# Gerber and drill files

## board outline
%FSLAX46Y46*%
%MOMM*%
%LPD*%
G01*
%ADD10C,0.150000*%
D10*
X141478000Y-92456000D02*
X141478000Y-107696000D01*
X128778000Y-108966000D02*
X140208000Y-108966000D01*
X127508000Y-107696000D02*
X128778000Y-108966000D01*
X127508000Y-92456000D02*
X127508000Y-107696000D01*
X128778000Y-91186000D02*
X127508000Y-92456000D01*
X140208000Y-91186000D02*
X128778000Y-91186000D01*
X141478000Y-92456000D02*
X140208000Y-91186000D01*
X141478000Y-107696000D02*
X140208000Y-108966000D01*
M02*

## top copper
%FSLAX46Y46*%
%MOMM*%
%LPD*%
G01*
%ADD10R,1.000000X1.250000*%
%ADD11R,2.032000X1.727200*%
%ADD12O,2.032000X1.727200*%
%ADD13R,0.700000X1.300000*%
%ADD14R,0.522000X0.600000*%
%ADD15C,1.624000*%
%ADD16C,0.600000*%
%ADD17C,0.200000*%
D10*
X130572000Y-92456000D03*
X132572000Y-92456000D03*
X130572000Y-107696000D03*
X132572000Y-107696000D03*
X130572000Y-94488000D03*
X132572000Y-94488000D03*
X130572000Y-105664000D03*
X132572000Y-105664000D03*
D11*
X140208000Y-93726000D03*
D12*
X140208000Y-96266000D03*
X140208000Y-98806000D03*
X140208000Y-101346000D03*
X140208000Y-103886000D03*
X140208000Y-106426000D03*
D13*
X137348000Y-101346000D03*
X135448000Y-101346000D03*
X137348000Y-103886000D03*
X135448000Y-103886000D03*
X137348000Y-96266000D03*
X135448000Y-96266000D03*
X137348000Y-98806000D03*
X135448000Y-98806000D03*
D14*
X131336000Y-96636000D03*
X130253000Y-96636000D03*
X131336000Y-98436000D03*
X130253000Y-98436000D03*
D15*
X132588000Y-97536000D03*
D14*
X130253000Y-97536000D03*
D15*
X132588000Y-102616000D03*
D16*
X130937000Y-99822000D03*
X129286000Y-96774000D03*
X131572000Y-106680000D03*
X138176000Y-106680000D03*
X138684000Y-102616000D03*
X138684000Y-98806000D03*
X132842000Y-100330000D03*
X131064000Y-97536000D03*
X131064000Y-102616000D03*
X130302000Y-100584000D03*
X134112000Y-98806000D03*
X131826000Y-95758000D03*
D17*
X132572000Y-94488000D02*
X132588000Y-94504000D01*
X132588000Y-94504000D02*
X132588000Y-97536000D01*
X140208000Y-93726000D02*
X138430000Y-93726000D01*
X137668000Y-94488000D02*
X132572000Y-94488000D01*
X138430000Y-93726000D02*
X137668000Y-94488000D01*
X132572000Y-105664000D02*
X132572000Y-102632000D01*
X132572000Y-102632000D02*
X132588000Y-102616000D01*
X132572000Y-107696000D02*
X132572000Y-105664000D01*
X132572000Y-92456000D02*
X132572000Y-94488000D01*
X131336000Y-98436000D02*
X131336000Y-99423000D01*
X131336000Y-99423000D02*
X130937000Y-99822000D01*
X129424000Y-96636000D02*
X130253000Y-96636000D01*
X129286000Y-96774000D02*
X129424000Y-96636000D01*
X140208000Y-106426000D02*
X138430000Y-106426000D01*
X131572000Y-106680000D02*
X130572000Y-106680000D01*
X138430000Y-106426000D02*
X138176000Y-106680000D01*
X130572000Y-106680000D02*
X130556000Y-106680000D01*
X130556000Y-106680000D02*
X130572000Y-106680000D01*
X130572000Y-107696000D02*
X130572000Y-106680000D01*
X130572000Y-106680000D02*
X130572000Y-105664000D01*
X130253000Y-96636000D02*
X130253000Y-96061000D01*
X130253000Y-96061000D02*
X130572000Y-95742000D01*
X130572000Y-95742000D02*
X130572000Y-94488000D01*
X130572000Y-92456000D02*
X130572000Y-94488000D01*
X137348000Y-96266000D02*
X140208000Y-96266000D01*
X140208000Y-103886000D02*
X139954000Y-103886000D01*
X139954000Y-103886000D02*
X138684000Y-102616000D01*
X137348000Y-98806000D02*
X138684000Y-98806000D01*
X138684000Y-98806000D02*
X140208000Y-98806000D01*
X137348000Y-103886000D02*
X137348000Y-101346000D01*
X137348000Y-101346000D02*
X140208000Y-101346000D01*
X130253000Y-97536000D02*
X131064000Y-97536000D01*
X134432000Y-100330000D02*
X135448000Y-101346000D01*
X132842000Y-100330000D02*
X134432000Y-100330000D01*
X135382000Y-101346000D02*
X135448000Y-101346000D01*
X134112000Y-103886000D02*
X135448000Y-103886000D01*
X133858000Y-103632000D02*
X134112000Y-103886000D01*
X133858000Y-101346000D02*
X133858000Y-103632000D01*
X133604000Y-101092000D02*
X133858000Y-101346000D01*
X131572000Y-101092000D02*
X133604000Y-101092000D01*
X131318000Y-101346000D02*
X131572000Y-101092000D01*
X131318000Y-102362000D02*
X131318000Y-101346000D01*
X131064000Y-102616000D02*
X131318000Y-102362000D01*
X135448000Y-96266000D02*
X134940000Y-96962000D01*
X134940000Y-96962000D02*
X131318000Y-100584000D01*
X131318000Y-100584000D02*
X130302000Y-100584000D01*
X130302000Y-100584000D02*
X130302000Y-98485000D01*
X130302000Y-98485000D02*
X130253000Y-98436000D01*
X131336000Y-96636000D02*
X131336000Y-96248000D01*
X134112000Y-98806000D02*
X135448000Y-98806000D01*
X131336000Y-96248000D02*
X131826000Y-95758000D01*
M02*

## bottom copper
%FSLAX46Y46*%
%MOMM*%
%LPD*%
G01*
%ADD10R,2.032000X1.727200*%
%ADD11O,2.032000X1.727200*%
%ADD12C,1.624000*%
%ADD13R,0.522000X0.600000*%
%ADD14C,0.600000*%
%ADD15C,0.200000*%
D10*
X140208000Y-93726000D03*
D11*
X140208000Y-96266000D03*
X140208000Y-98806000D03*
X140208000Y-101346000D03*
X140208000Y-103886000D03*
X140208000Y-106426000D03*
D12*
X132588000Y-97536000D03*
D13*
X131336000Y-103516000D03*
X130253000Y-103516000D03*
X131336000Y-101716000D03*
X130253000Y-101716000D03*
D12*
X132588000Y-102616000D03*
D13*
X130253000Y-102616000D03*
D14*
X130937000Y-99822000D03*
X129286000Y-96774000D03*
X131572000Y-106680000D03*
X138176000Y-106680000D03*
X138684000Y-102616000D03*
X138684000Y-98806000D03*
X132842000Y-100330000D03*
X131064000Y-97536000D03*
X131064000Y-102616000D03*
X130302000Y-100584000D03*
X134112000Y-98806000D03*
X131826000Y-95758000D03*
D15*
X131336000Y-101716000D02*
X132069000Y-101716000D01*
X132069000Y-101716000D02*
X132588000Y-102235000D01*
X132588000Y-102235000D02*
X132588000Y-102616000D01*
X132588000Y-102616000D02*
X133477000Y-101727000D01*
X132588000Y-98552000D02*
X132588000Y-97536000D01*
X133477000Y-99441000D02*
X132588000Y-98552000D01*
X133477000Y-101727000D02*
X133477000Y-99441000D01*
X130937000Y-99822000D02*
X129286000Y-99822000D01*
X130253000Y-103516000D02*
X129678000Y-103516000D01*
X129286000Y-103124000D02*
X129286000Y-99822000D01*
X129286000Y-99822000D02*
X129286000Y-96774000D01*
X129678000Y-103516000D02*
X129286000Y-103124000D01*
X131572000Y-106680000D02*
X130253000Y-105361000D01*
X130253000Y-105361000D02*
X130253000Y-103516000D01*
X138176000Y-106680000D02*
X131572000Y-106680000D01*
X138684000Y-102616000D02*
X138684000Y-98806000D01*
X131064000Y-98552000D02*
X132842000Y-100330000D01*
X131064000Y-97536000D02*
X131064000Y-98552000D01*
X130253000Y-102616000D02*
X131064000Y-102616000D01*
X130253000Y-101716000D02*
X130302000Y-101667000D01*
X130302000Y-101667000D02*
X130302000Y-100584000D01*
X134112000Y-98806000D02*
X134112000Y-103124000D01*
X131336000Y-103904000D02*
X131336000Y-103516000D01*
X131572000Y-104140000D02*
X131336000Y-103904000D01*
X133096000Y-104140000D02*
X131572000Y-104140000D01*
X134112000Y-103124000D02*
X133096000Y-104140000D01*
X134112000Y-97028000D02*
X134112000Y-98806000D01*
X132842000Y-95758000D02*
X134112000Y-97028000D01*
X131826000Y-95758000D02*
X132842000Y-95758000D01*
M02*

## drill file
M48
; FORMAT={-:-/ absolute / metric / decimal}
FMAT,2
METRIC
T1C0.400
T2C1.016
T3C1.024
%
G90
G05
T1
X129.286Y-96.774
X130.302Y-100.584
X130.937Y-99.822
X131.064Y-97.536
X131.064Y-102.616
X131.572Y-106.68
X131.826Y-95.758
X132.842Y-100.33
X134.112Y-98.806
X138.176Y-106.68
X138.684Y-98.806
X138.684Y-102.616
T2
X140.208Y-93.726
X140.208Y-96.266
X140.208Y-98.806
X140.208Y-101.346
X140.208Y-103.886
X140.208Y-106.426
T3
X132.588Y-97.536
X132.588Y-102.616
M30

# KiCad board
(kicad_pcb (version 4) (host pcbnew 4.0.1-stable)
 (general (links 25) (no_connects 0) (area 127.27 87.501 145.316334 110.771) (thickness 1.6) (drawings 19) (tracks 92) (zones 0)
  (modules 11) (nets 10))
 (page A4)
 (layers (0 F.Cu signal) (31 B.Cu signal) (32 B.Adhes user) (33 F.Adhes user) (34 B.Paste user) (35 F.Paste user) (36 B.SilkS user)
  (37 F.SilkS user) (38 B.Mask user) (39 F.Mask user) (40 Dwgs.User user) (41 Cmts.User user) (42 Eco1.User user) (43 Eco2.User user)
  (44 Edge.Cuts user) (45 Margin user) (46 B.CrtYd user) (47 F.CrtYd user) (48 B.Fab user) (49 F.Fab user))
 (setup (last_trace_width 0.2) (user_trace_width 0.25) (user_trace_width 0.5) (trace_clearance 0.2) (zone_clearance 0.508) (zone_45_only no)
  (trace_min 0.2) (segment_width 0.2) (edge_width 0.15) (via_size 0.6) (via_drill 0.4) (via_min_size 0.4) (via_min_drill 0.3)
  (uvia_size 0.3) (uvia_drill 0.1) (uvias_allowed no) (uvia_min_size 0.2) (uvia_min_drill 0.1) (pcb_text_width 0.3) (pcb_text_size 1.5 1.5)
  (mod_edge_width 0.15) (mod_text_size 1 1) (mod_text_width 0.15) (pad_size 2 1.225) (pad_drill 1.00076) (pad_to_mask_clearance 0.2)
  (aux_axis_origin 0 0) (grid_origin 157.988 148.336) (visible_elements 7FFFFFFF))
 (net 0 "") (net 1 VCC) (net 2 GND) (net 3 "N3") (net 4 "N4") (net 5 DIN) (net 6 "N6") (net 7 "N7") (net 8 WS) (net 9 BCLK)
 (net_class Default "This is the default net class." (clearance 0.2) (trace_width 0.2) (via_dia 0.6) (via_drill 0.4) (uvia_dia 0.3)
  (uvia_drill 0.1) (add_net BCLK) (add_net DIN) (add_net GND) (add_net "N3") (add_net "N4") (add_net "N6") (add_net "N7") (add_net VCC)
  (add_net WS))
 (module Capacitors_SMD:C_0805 (layer F.Cu) (at 131.572 92.456)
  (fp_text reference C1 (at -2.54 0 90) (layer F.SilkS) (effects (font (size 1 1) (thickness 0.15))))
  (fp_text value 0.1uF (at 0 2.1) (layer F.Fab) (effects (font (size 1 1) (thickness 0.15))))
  (pad 1 smd rect (at -1 0) (size 1 1.25) (layers F.Cu F.Paste F.Mask) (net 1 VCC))
  (pad 2 smd rect (at 1 0) (size 1 1.25) (layers F.Cu F.Paste F.Mask) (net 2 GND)))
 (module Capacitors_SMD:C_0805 (layer F.Cu) (at 131.572 107.696)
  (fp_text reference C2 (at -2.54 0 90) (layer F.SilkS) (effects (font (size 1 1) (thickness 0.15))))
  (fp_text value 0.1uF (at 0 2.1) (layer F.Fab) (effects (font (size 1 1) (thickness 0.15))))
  (pad 1 smd rect (at -1 0) (size 1 1.25) (layers F.Cu F.Paste F.Mask) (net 1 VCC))
  (pad 2 smd rect (at 1 0) (size 1 1.25) (layers F.Cu F.Paste F.Mask) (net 2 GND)))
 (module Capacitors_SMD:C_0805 (layer F.Cu) (at 131.572 94.488)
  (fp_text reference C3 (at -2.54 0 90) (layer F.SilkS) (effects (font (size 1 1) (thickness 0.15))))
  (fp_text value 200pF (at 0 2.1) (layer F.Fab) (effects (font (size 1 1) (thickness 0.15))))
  (pad 1 smd rect (at -1 0) (size 1 1.25) (layers F.Cu F.Paste F.Mask) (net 1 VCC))
  (pad 2 smd rect (at 1 0) (size 1 1.25) (layers F.Cu F.Paste F.Mask) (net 2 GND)))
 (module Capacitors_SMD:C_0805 (layer F.Cu) (at 131.572 105.664)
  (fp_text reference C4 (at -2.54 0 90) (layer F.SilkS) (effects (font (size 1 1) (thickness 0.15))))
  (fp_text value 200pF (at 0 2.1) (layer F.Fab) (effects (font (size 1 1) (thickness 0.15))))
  (pad 1 smd rect (at -1 0) (size 1 1.25) (layers F.Cu F.Paste F.Mask) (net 1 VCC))
  (pad 2 smd rect (at 1 0) (size 1 1.25) (layers F.Cu F.Paste F.Mask) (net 2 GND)))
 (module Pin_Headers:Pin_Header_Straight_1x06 (layer F.Cu) (at 140.208 93.726)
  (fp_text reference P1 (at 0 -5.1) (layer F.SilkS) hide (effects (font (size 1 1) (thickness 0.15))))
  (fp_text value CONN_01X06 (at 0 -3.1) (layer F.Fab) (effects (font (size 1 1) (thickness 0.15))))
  (pad 1 thru_hole rect (at 0 0) (size 2.032 1.7272) (drill 1.016) (layers *.Cu *.Mask F.SilkS) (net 2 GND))
  (pad 2 thru_hole oval (at 0 2.54) (size 2.032 1.7272) (drill 1.016) (layers *.Cu *.Mask F.SilkS) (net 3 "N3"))
  (pad 3 thru_hole oval (at 0 5.08) (size 2.032 1.7272) (drill 1.016) (layers *.Cu *.Mask F.SilkS) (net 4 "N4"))
  (pad 4 thru_hole oval (at 0 7.62) (size 2.032 1.7272) (drill 1.016) (layers *.Cu *.Mask F.SilkS) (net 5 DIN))
  (pad 5 thru_hole oval (at 0 10.16) (size 2.032 1.7272) (drill 1.016) (layers *.Cu *.Mask F.SilkS) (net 4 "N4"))
  (pad 6 thru_hole oval (at 0 12.7) (size 2.032 1.7272) (drill 1.016) (layers *.Cu *.Mask F.SilkS) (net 1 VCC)))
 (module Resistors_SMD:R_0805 (layer F.Cu) (at 136.398 101.346 180)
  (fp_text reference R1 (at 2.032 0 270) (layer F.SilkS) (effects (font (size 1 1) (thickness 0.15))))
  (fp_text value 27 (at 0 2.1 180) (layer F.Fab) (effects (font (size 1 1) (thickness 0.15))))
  (pad 1 smd rect (at -0.95 0 180) (size 0.7 1.3) (layers F.Cu F.Paste F.Mask) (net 5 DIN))
  (pad 2 smd rect (at 0.95 0 180) (size 0.7 1.3) (layers F.Cu F.Paste F.Mask) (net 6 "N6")))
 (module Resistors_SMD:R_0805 (layer F.Cu) (at 136.398 103.886 180)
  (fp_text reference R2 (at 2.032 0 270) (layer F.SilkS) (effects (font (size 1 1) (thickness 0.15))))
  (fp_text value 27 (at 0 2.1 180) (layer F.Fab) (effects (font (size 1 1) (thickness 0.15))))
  (pad 1 smd rect (at -0.95 0 180) (size 0.7 1.3) (layers F.Cu F.Paste F.Mask) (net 5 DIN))
  (pad 2 smd rect (at 0.95 0 180) (size 0.7 1.3) (layers F.Cu F.Paste F.Mask) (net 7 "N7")))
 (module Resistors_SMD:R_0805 (layer F.Cu) (at 136.398 96.266 180)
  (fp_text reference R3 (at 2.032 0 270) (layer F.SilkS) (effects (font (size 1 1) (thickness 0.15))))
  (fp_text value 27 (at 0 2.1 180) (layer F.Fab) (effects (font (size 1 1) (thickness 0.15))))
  (pad 1 smd rect (at -0.95 0 180) (size 0.7 1.3) (layers F.Cu F.Paste F.Mask) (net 3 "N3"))
  (pad 2 smd rect (at 0.95 0 180) (size 0.7 1.3) (layers F.Cu F.Paste F.Mask) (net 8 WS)))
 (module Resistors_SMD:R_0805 (layer F.Cu) (at 136.398 98.806 180)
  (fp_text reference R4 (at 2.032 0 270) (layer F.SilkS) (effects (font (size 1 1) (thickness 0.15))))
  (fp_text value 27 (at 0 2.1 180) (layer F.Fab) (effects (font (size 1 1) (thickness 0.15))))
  (pad 1 smd rect (at -0.95 0 180) (size 0.7 1.3) (layers F.Cu F.Paste F.Mask) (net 4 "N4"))
  (pad 2 smd rect (at 0.95 0 180) (size 0.7 1.3) (layers F.Cu F.Paste F.Mask) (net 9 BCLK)))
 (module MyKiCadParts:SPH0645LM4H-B (layer F.Cu) (at 132.588 97.536 90)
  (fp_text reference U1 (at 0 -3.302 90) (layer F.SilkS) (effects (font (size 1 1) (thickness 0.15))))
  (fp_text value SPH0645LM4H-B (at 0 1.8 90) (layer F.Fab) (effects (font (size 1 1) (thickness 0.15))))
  (pad 4 smd rect (at 0.9 -1.252 90) (size 0.6 0.522) (layers F.Cu F.Paste F.Mask) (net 9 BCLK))
  (pad 5 smd rect (at 0.9 -2.335 90) (size 0.6 0.522) (layers F.Cu F.Paste F.Mask) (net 1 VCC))
  (pad 2 smd rect (at -0.9 -1.252 90) (size 0.6 0.522) (layers F.Cu F.Paste F.Mask) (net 1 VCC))
  (pad 1 smd rect (at -0.9 -2.335 90) (size 0.6 0.522) (layers F.Cu F.Paste F.Mask) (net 8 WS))
  (pad 3 thru_hole circle (at 0 0 90) (size 1.624 1.624) (drill 1.024) (layers *.Cu *.Mask F.SilkS) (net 2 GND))
  (pad 6 smd rect (at 0 -2.335 90) (size 0.6 0.522) (layers F.Cu F.Paste F.Mask) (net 6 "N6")))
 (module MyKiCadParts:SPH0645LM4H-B (layer B.Cu) (at 132.588 102.616 270)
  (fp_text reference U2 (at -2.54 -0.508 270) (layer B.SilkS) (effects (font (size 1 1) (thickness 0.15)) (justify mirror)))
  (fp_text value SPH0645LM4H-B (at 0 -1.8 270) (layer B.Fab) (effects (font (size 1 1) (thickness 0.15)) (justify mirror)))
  (pad 4 smd rect (at 0.9 1.252 270) (size 0.6 0.522) (layers B.Cu B.Paste B.Mask) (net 9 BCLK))
  (pad 5 smd rect (at 0.9 2.335 270) (size 0.6 0.522) (layers B.Cu B.Paste B.Mask) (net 1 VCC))
  (pad 2 smd rect (at -0.9 1.252 270) (size 0.6 0.522) (layers B.Cu B.Paste B.Mask) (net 2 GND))
  (pad 1 smd rect (at -0.9 2.335 270) (size 0.6 0.522) (layers B.Cu B.Paste B.Mask) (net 8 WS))
  (pad 3 thru_hole circle (at 0 0 270) (size 1.624 1.624) (drill 1.024) (layers *.Cu *.Mask B.SilkS) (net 2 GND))
  (pad 6 smd rect (at 0 2.335 270) (size 0.6 0.522) (layers B.Cu B.Paste B.Mask) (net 7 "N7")))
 (gr_line (start 141.478 92.456) (end 141.478 107.696) (angle 90) (layer Edge.Cuts) (width 0.15))
 (gr_line (start 128.778 108.966) (end 140.208 108.966) (angle 90) (layer Edge.Cuts) (width 0.15))
 (gr_line (start 127.508 107.696) (end 128.778 108.966) (angle 90) (layer Edge.Cuts) (width 0.15))
 (gr_line (start 127.508 92.456) (end 127.508 107.696) (angle 90) (layer Edge.Cuts) (width 0.15))
 (gr_line (start 128.778 91.186) (end 127.508 92.456) (angle 90) (layer Edge.Cuts) (width 0.15))
 (gr_line (start 140.208 91.186) (end 128.778 91.186) (angle 90) (layer Edge.Cuts) (width 0.15))
 (gr_line (start 141.478 92.456) (end 140.208 91.186) (angle 90) (layer Edge.Cuts) (width 0.15))
 (gr_line (start 141.478 107.696) (end 140.208 108.966) (angle 90) (layer Edge.Cuts) (width 0.15))
 (segment (start 131.336 101.716) (end 132.069 101.716) (width 0.2) (layer B.Cu) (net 2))
 (segment (start 132.069 101.716) (end 132.588 102.235) (width 0.2) (layer B.Cu) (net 2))
 (segment (start 132.588 102.235) (end 132.588 102.616) (width 0.2) (layer B.Cu) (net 2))
 (segment (start 132.588 102.616) (end 133.477 101.727) (width 0.2) (layer B.Cu) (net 2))
 (segment (start 132.588 98.552) (end 132.588 97.536) (width 0.2) (layer B.Cu) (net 2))
 (segment (start 133.477 99.441) (end 132.588 98.552) (width 0.2) (layer B.Cu) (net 2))
 (segment (start 133.477 101.727) (end 133.477 99.441) (width 0.2) (layer B.Cu) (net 2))
 (segment (start 132.572 94.488) (end 132.588 94.504) (width 0.2) (layer F.Cu) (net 2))
 (segment (start 132.588 94.504) (end 132.588 97.536) (width 0.2) (layer F.Cu) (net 2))
 (segment (start 140.208 93.726) (end 138.43 93.726) (width 0.2) (layer F.Cu) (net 2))
 (segment (start 137.668 94.488) (end 132.572 94.488) (width 0.2) (layer F.Cu) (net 2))
 (segment (start 138.43 93.726) (end 137.668 94.488) (width 0.2) (layer F.Cu) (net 2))
 (segment (start 132.572 105.664) (end 132.572 102.632) (width 0.2) (layer F.Cu) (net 2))
 (segment (start 132.572 102.632) (end 132.588 102.616) (width 0.2) (layer F.Cu) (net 2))
 (segment (start 132.572 107.696) (end 132.572 105.664) (width 0.2) (layer F.Cu) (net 2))
 (segment (start 132.572 92.456) (end 132.572 94.488) (width 0.2) (layer F.Cu) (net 2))
 (segment (start 131.336 98.436) (end 131.336 99.423) (width 0.2) (layer F.Cu) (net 1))
 (segment (start 130.937 99.822) (end 129.286 99.822) (width 0.2) (layer B.Cu) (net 1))
 (via (at 130.937 99.822) (size 0.6) (drill 0.4) (layers F.Cu B.Cu) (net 1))
 (segment (start 131.336 99.423) (end 130.937 99.822) (width 0.2) (layer F.Cu) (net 1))
 (segment (start 130.253 103.516) (end 129.678 103.516) (width 0.2) (layer B.Cu) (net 1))
 (segment (start 129.424 96.636) (end 130.253 96.636) (width 0.2) (layer F.Cu) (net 1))
 (segment (start 129.286 96.774) (end 129.424 96.636) (width 0.2) (layer F.Cu) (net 1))
 (via (at 129.286 96.774) (size 0.6) (drill 0.4) (layers F.Cu B.Cu) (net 1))
 (segment (start 129.286 103.124) (end 129.286 99.822) (width 0.2) (layer B.Cu) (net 1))
 (segment (start 129.286 99.822) (end 129.286 96.774) (width 0.2) (layer B.Cu) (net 1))
 (segment (start 129.678 103.516) (end 129.286 103.124) (width 0.2) (layer B.Cu) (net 1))
 (segment (start 131.572 106.68) (end 130.253 105.361) (width 0.2) (layer B.Cu) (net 1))
 (segment (start 130.253 105.361) (end 130.253 103.516) (width 0.2) (layer B.Cu) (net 1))
 (segment (start 140.208 106.426) (end 138.43 106.426) (width 0.2) (layer F.Cu) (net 1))
 (segment (start 131.572 106.68) (end 130.572 106.68) (width 0.2) (layer F.Cu) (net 1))
 (via (at 131.572 106.68) (size 0.6) (drill 0.4) (layers F.Cu B.Cu) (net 1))
 (segment (start 138.176 106.68) (end 131.572 106.68) (width 0.2) (layer B.Cu) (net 1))
 (via (at 138.176 106.68) (size 0.6) (drill 0.4) (layers F.Cu B.Cu) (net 1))
 (segment (start 138.43 106.426) (end 138.176 106.68) (width 0.2) (layer F.Cu) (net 1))
 (segment (start 130.572 106.68) (end 130.556 106.68) (width 0.2) (layer F.Cu) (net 1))
 (segment (start 130.556 106.68) (end 130.572 106.68) (width 0.2) (layer F.Cu) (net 1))
 (segment (start 130.572 107.696) (end 130.572 106.68) (width 0.2) (layer F.Cu) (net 1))
 (segment (start 130.572 106.68) (end 130.572 105.664) (width 0.2) (layer F.Cu) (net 1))
 (segment (start 130.253 96.636) (end 130.253 96.061) (width 0.2) (layer F.Cu) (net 1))
 (segment (start 130.253 96.061) (end 130.572 95.742) (width 0.2) (layer F.Cu) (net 1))
 (segment (start 130.572 95.742) (end 130.572 94.488) (width 0.2) (layer F.Cu) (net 1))
 (segment (start 130.572 92.456) (end 130.572 94.488) (width 0.2) (layer F.Cu) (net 1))
 (segment (start 137.348 96.266) (end 140.208 96.266) (width 0.2) (layer F.Cu) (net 3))
 (segment (start 140.208 103.886) (end 139.954 103.886) (width 0.2) (layer F.Cu) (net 4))
 (segment (start 139.954 103.886) (end 138.684 102.616) (width 0.2) (layer F.Cu) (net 4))
 (via (at 138.684 102.616) (size 0.6) (drill 0.4) (layers F.Cu B.Cu) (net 4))
 (segment (start 138.684 102.616) (end 138.684 98.806) (width 0.2) (layer B.Cu) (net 4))
 (via (at 138.684 98.806) (size 0.6) (drill 0.4) (layers F.Cu B.Cu) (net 4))
 (segment (start 137.348 98.806) (end 138.684 98.806) (width 0.2) (layer F.Cu) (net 4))
 (segment (start 138.684 98.806) (end 140.208 98.806) (width 0.2) (layer F.Cu) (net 4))
 (segment (start 137.348 103.886) (end 137.348 101.346) (width 0.2) (layer F.Cu) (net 5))
 (segment (start 137.348 101.346) (end 140.208 101.346) (width 0.2) (layer F.Cu) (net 5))
 (segment (start 130.253 97.536) (end 131.064 97.536) (width 0.2) (layer F.Cu) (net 6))
 (segment (start 134.432 100.33) (end 135.448 101.346) (width 0.2) (layer F.Cu) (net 6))
 (segment (start 132.842 100.33) (end 134.432 100.33) (width 0.2) (layer F.Cu) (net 6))
 (via (at 132.842 100.33) (size 0.6) (drill 0.4) (layers F.Cu B.Cu) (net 6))
 (segment (start 131.064 98.552) (end 132.842 100.33) (width 0.2) (layer B.Cu) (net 6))
 (segment (start 131.064 97.536) (end 131.064 98.552) (width 0.2) (layer B.Cu) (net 6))
 (via (at 131.064 97.536) (size 0.6) (drill 0.4) (layers F.Cu B.Cu) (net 6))
 (segment (start 135.382 101.346) (end 135.448 101.346) (width 0.2) (layer F.Cu) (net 6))
 (segment (start 130.253 102.616) (end 131.064 102.616) (width 0.2) (layer B.Cu) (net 7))
 (segment (start 134.112 103.886) (end 135.448 103.886) (width 0.2) (layer F.Cu) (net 7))
 (segment (start 133.858 103.632) (end 134.112 103.886) (width 0.2) (layer F.Cu) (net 7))
 (segment (start 133.858 101.346) (end 133.858 103.632) (width 0.2) (layer F.Cu) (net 7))
 (segment (start 133.604 101.092) (end 133.858 101.346) (width 0.2) (layer F.Cu) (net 7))
 (segment (start 131.572 101.092) (end 133.604 101.092) (width 0.2) (layer F.Cu) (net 7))
 (segment (start 131.318 101.346) (end 131.572 101.092) (width 0.2) (layer F.Cu) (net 7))
 (segment (start 131.318 102.362) (end 131.318 101.346) (width 0.2) (layer F.Cu) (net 7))
 (segment (start 131.064 102.616) (end 131.318 102.362) (width 0.2) (layer F.Cu) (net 7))
 (via (at 131.064 102.616) (size 0.6) (drill 0.4) (layers F.Cu B.Cu) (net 7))
 (segment (start 135.448 96.266) (end 134.94 96.962) (width 0.2) (layer F.Cu) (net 8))
 (segment (start 134.94 96.962) (end 131.318 100.584) (width 0.2) (layer F.Cu) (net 8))
 (segment (start 131.318 100.584) (end 130.302 100.584) (width 0.2) (layer F.Cu) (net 8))
 (segment (start 130.253 101.716) (end 130.302 101.667) (width 0.2) (layer B.Cu) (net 8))
 (segment (start 130.302 101.667) (end 130.302 100.584) (width 0.2) (layer B.Cu) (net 8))
 (via (at 130.302 100.584) (size 0.6) (drill 0.4) (layers F.Cu B.Cu) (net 8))
 (segment (start 130.302 100.584) (end 130.302 98.485) (width 0.2) (layer F.Cu) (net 8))
 (segment (start 130.302 98.485) (end 130.253 98.436) (width 0.2) (layer F.Cu) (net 8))
 (segment (start 134.112 98.806) (end 134.112 103.124) (width 0.2) (layer B.Cu) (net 9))
 (segment (start 131.336 103.904) (end 131.336 103.516) (width 0.2) (layer B.Cu) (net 9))
 (segment (start 131.572 104.14) (end 131.336 103.904) (width 0.2) (layer B.Cu) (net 9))
 (segment (start 133.096 104.14) (end 131.572 104.14) (width 0.2) (layer B.Cu) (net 9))
 (segment (start 134.112 103.124) (end 133.096 104.14) (width 0.2) (layer B.Cu) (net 9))
 (segment (start 131.336 96.636) (end 131.336 96.248) (width 0.2) (layer F.Cu) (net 9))
 (segment (start 134.112 98.806) (end 135.448 98.806) (width 0.2) (layer F.Cu) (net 9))
 (via (at 134.112 98.806) (size 0.6) (drill 0.4) (layers F.Cu B.Cu) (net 9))
 (segment (start 134.112 97.028) (end 134.112 98.806) (width 0.2) (layer B.Cu) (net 9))
 (segment (start 132.842 95.758) (end 134.112 97.028) (width 0.2) (layer B.Cu) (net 9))
 (segment (start 131.826 95.758) (end 132.842 95.758) (width 0.2) (layer B.Cu) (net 9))
 (via (at 131.826 95.758) (size 0.6) (drill 0.4) (layers F.Cu B.Cu) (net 9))
 (segment (start 131.336 96.248) (end 131.826 95.758) (width 0.2) (layer F.Cu) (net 9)))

